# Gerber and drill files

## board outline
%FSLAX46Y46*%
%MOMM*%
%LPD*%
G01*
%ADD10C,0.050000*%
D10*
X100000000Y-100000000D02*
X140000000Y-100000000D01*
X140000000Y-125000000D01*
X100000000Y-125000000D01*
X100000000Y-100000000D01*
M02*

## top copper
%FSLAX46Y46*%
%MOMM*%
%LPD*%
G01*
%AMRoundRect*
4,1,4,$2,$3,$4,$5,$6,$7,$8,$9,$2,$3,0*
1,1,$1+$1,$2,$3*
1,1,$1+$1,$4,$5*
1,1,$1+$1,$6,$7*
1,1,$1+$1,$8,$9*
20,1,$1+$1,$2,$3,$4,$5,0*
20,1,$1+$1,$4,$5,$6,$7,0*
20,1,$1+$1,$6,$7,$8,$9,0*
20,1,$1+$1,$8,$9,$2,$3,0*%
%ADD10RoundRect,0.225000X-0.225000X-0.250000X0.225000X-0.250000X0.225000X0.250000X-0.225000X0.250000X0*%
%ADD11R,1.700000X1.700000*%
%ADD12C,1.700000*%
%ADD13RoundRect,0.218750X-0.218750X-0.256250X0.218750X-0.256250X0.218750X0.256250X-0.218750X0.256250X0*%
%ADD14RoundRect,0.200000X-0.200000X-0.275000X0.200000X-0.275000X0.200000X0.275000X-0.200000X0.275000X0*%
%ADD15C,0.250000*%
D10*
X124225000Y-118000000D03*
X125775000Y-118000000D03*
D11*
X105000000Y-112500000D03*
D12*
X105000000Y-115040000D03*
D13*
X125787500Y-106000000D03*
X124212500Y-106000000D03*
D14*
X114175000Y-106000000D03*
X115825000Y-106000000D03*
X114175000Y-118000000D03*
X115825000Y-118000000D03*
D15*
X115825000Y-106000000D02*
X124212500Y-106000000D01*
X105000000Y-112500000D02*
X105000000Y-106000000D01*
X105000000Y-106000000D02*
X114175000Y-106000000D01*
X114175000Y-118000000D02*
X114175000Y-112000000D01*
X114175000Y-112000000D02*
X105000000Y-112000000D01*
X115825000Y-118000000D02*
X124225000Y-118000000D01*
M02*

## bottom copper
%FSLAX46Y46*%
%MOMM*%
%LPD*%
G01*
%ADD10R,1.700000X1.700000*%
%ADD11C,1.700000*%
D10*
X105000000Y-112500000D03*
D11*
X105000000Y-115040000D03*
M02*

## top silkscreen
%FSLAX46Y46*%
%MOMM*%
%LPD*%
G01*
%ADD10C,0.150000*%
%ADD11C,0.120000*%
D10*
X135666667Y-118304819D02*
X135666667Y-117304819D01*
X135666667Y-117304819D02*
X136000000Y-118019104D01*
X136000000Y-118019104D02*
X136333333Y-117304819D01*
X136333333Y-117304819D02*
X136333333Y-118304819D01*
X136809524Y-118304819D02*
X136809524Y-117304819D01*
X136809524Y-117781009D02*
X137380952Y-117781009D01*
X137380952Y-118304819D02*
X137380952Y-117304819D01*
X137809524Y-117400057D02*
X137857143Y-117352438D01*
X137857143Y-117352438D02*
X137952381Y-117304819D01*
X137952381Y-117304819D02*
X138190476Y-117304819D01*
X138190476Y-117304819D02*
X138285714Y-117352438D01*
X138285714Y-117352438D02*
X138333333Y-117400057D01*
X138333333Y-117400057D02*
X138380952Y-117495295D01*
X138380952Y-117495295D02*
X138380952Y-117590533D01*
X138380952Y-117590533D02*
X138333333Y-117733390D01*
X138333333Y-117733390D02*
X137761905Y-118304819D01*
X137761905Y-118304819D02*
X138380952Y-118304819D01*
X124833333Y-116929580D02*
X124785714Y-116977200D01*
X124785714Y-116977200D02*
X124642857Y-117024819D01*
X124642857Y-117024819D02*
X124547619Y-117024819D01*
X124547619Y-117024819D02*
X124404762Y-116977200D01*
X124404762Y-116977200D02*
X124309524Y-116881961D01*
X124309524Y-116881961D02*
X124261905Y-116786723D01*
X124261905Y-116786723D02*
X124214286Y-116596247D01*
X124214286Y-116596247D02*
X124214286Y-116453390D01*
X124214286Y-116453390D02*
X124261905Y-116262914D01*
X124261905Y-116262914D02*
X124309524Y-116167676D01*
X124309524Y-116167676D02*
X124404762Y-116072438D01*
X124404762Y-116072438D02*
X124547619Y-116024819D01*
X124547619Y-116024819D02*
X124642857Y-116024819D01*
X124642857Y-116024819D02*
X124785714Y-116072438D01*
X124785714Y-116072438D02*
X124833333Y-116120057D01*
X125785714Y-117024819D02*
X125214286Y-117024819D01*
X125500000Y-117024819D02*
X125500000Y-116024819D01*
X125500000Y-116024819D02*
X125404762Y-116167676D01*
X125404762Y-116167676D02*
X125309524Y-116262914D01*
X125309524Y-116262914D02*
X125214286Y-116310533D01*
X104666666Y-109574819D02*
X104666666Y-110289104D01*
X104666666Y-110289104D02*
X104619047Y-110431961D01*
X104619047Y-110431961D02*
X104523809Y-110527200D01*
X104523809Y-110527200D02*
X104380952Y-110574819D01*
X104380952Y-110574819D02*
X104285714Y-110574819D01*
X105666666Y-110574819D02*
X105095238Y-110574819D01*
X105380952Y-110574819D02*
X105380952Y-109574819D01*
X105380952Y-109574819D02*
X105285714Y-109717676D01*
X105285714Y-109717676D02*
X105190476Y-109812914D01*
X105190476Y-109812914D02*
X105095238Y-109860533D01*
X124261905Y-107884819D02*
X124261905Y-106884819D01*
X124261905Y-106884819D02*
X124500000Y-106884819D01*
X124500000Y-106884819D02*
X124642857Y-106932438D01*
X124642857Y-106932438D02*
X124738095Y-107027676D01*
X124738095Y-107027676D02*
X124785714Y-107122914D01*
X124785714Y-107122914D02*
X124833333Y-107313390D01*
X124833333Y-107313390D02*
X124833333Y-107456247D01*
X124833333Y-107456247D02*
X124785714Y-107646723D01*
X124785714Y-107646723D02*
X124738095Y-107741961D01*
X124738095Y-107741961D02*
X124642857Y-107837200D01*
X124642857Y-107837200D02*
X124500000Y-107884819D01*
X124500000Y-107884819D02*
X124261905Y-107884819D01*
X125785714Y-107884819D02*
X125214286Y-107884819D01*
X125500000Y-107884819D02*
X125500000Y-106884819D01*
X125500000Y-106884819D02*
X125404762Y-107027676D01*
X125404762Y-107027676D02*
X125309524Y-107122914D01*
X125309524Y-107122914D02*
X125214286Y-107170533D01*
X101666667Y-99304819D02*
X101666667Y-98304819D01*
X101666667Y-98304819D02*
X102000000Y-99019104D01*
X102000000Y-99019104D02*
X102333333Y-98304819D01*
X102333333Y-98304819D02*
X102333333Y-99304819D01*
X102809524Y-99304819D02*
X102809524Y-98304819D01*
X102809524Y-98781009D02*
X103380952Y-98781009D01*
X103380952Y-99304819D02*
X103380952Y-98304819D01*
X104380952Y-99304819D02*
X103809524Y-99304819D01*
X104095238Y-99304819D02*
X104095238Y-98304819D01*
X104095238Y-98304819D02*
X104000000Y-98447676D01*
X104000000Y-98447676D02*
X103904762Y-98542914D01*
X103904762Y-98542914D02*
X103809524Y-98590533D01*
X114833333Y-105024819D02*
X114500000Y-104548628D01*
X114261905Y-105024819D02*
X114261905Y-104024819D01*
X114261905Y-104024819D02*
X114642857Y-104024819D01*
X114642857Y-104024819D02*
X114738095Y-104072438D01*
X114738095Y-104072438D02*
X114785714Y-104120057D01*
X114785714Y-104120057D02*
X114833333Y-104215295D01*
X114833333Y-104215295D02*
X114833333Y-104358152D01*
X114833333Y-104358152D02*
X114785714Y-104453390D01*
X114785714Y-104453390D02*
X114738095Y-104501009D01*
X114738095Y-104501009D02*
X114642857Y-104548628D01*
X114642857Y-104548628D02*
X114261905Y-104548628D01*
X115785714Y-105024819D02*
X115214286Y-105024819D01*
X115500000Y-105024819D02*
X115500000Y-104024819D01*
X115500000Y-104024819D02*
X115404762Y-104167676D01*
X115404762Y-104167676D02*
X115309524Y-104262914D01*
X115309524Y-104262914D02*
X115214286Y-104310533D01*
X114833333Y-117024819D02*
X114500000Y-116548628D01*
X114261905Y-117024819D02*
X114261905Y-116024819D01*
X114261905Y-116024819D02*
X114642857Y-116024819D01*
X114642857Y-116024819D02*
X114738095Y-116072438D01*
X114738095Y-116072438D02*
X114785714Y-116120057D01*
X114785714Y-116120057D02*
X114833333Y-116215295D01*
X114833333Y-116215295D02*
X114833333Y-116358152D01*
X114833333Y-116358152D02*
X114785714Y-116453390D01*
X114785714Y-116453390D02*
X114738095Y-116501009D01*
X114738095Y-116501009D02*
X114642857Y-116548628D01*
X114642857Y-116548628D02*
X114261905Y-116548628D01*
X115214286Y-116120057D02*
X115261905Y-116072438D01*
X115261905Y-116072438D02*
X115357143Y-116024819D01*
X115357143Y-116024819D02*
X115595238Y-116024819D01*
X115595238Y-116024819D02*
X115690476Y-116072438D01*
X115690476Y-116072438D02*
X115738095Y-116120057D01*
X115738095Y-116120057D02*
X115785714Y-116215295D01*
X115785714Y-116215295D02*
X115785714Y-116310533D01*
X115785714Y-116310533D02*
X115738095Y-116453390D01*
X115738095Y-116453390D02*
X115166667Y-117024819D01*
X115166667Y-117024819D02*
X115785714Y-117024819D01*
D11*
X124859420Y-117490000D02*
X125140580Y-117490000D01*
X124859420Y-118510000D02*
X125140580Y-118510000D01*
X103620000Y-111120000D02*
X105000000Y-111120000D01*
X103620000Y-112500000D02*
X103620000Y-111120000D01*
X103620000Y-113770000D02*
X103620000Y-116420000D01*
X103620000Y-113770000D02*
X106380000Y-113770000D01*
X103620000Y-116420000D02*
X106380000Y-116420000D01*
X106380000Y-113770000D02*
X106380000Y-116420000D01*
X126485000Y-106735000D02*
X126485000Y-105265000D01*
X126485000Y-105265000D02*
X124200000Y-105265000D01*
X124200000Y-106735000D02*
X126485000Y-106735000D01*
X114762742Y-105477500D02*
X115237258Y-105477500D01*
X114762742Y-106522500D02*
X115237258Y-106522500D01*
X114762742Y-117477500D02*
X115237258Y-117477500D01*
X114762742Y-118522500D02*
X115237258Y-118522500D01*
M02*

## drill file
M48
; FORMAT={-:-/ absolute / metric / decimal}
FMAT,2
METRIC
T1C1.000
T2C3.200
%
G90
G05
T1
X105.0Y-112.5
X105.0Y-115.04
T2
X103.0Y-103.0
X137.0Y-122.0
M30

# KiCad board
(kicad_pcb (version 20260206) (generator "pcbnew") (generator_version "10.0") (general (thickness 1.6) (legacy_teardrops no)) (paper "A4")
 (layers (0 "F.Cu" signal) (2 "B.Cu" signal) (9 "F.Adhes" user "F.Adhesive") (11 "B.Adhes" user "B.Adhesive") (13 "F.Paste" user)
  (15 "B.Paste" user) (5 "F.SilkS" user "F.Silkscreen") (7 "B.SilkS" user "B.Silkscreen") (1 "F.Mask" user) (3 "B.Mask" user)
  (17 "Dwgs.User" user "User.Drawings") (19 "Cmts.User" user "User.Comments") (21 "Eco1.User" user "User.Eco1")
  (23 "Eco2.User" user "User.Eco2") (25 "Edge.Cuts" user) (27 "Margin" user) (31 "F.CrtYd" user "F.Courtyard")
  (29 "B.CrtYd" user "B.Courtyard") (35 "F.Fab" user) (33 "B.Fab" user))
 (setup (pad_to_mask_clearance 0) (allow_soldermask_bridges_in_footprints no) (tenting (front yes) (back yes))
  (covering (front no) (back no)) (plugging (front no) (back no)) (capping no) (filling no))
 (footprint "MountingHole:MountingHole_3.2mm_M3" (layer "F.Cu") (at 137 122)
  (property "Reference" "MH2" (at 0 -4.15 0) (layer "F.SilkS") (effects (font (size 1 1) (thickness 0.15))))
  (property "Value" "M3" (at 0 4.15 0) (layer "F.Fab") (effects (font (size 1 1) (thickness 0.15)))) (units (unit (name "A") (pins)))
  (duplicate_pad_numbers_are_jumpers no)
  (pad "" np_thru_hole circle (at 0 0) (size 3.2 3.2) (drill 3.2) (layers "*.Cu" "*.Mask")))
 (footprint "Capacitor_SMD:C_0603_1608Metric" (layer "F.Cu") (at 125 118)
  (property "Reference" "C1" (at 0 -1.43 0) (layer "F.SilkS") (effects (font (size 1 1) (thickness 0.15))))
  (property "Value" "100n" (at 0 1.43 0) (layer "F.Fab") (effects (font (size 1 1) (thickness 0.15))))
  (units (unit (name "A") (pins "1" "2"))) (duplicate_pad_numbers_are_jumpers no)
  (fp_line (start -0.14058 -0.51) (end 0.14058 -0.51) (stroke (width 0.12) (type solid)) (layer "F.SilkS"))
  (fp_line (start -0.14058 0.51) (end 0.14058 0.51) (stroke (width 0.12) (type solid)) (layer "F.SilkS"))
  (pad "1" smd roundrect (at -0.775 0) (size 0.9 0.95) (layers "F.Cu" "F.Mask" "F.Paste") (roundrect_rratio 0.25) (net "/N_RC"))
  (pad "2" smd roundrect (at 0.775 0) (size 0.9 0.95) (layers "F.Cu" "F.Mask" "F.Paste") (roundrect_rratio 0.25) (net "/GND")))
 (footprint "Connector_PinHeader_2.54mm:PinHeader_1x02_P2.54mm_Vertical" (layer "F.Cu") (at 105 112.5)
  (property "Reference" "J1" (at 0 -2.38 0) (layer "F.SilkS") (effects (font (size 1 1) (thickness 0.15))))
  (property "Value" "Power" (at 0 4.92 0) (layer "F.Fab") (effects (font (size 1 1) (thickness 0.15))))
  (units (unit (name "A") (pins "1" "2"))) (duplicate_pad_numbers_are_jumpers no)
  (fp_line (start -1.38 -1.38) (end 0 -1.38) (stroke (width 0.12) (type solid)) (layer "F.SilkS"))
  (fp_line (start -1.38 0) (end -1.38 -1.38) (stroke (width 0.12) (type solid)) (layer "F.SilkS"))
  (fp_line (start -1.38 1.27) (end -1.38 3.92) (stroke (width 0.12) (type solid)) (layer "F.SilkS"))
  (fp_line (start -1.38 1.27) (end 1.38 1.27) (stroke (width 0.12) (type solid)) (layer "F.SilkS"))
  (fp_line (start -1.38 3.92) (end 1.38 3.92) (stroke (width 0.12) (type solid)) (layer "F.SilkS"))
  (fp_line (start 1.38 1.27) (end 1.38 3.92) (stroke (width 0.12) (type solid)) (layer "F.SilkS"))
  (pad "1" thru_hole rect (at 0 0) (size 1.7 1.7) (drill 1) (layers "*.Cu" "*.Mask") (remove_unused_layers no) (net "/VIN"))
  (pad "2" thru_hole circle (at 0 2.54) (size 1.7 1.7) (drill 1) (layers "*.Cu" "*.Mask") (remove_unused_layers no) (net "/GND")))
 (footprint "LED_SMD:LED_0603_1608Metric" (layer "F.Cu") (at 125 106 180)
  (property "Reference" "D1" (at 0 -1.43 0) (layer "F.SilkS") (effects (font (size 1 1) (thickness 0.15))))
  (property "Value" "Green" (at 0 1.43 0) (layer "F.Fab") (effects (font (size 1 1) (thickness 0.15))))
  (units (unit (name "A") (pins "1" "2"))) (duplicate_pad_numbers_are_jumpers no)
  (fp_line (start -1.485 -0.735) (end -1.485 0.735) (stroke (width 0.12) (type solid)) (layer "F.SilkS"))
  (fp_line (start -1.485 0.735) (end 0.8 0.735) (stroke (width 0.12) (type solid)) (layer "F.SilkS"))
  (fp_line (start 0.8 -0.735) (end -1.485 -0.735) (stroke (width 0.12) (type solid)) (layer "F.SilkS"))
  (pad "1" smd roundrect (at -0.7875 0) (size 0.875 0.95) (layers "F.Cu" "F.Mask" "F.Paste") (roundrect_rratio 0.25) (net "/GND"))
  (pad "2" smd roundrect (at 0.7875 0) (size 0.875 0.95) (layers "F.Cu" "F.Mask" "F.Paste") (roundrect_rratio 0.25) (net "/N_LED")))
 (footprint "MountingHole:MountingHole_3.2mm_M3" (layer "F.Cu") (at 103 103)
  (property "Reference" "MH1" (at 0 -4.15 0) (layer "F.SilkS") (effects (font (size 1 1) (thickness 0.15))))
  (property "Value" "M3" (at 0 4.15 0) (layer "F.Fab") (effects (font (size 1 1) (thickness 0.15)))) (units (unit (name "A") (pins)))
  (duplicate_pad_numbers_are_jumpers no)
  (pad "" np_thru_hole circle (at 0 0) (size 3.2 3.2) (drill 3.2) (layers "*.Cu" "*.Mask")))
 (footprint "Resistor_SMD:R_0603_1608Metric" (layer "F.Cu") (at 115 106)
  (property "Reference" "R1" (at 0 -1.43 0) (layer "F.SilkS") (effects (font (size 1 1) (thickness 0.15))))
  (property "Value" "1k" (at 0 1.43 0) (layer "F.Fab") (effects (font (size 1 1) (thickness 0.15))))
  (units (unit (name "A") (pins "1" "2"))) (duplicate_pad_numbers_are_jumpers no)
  (fp_line (start -0.237258 -0.5225) (end 0.237258 -0.5225) (stroke (width 0.12) (type solid)) (layer "F.SilkS"))
  (fp_line (start -0.237258 0.5225) (end 0.237258 0.5225) (stroke (width 0.12) (type solid)) (layer "F.SilkS"))
  (pad "1" smd roundrect (at -0.825 0) (size 0.8 0.95) (layers "F.Cu" "F.Mask" "F.Paste") (roundrect_rratio 0.25) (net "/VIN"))
  (pad "2" smd roundrect (at 0.825 0) (size 0.8 0.95) (layers "F.Cu" "F.Mask" "F.Paste") (roundrect_rratio 0.25) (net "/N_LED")))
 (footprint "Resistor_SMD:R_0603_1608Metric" (layer "F.Cu") (at 115 118)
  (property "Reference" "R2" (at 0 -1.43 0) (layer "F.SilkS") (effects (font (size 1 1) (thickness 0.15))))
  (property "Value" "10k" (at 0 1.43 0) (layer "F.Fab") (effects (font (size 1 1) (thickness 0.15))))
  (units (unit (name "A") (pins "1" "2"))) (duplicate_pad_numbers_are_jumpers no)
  (fp_line (start -0.237258 -0.5225) (end 0.237258 -0.5225) (stroke (width 0.12) (type solid)) (layer "F.SilkS"))
  (fp_line (start -0.237258 0.5225) (end 0.237258 0.5225) (stroke (width 0.12) (type solid)) (layer "F.SilkS"))
  (pad "1" smd roundrect (at -0.825 0) (size 0.8 0.95) (layers "F.Cu" "F.Mask" "F.Paste") (roundrect_rratio 0.25) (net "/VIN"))
  (pad "2" smd roundrect (at 0.825 0) (size 0.8 0.95) (layers "F.Cu" "F.Mask" "F.Paste") (roundrect_rratio 0.25) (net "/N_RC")))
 (gr_rect (start 100 100) (end 140 125) (stroke (width 0.05) (type default)) (fill no) (layer "Edge.Cuts"))
 (segment (start 115.825 106) (end 124.2125 106) (width 0.25) (layer "F.Cu") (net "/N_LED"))
 (segment (start 105 112.5) (end 105 106) (width 0.25) (layer "F.Cu") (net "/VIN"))
 (segment (start 105 106) (end 114.175 106) (width 0.25) (layer "F.Cu") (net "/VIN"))
 (segment (start 114.175 118) (end 114.175 112) (width 0.25) (layer "F.Cu") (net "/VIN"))
 (segment (start 114.175 112) (end 105 112) (width 0.25) (layer "F.Cu") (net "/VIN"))
 (segment (start 115.825 118) (end 124.225 118) (width 0.25) (layer "F.Cu") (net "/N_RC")))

